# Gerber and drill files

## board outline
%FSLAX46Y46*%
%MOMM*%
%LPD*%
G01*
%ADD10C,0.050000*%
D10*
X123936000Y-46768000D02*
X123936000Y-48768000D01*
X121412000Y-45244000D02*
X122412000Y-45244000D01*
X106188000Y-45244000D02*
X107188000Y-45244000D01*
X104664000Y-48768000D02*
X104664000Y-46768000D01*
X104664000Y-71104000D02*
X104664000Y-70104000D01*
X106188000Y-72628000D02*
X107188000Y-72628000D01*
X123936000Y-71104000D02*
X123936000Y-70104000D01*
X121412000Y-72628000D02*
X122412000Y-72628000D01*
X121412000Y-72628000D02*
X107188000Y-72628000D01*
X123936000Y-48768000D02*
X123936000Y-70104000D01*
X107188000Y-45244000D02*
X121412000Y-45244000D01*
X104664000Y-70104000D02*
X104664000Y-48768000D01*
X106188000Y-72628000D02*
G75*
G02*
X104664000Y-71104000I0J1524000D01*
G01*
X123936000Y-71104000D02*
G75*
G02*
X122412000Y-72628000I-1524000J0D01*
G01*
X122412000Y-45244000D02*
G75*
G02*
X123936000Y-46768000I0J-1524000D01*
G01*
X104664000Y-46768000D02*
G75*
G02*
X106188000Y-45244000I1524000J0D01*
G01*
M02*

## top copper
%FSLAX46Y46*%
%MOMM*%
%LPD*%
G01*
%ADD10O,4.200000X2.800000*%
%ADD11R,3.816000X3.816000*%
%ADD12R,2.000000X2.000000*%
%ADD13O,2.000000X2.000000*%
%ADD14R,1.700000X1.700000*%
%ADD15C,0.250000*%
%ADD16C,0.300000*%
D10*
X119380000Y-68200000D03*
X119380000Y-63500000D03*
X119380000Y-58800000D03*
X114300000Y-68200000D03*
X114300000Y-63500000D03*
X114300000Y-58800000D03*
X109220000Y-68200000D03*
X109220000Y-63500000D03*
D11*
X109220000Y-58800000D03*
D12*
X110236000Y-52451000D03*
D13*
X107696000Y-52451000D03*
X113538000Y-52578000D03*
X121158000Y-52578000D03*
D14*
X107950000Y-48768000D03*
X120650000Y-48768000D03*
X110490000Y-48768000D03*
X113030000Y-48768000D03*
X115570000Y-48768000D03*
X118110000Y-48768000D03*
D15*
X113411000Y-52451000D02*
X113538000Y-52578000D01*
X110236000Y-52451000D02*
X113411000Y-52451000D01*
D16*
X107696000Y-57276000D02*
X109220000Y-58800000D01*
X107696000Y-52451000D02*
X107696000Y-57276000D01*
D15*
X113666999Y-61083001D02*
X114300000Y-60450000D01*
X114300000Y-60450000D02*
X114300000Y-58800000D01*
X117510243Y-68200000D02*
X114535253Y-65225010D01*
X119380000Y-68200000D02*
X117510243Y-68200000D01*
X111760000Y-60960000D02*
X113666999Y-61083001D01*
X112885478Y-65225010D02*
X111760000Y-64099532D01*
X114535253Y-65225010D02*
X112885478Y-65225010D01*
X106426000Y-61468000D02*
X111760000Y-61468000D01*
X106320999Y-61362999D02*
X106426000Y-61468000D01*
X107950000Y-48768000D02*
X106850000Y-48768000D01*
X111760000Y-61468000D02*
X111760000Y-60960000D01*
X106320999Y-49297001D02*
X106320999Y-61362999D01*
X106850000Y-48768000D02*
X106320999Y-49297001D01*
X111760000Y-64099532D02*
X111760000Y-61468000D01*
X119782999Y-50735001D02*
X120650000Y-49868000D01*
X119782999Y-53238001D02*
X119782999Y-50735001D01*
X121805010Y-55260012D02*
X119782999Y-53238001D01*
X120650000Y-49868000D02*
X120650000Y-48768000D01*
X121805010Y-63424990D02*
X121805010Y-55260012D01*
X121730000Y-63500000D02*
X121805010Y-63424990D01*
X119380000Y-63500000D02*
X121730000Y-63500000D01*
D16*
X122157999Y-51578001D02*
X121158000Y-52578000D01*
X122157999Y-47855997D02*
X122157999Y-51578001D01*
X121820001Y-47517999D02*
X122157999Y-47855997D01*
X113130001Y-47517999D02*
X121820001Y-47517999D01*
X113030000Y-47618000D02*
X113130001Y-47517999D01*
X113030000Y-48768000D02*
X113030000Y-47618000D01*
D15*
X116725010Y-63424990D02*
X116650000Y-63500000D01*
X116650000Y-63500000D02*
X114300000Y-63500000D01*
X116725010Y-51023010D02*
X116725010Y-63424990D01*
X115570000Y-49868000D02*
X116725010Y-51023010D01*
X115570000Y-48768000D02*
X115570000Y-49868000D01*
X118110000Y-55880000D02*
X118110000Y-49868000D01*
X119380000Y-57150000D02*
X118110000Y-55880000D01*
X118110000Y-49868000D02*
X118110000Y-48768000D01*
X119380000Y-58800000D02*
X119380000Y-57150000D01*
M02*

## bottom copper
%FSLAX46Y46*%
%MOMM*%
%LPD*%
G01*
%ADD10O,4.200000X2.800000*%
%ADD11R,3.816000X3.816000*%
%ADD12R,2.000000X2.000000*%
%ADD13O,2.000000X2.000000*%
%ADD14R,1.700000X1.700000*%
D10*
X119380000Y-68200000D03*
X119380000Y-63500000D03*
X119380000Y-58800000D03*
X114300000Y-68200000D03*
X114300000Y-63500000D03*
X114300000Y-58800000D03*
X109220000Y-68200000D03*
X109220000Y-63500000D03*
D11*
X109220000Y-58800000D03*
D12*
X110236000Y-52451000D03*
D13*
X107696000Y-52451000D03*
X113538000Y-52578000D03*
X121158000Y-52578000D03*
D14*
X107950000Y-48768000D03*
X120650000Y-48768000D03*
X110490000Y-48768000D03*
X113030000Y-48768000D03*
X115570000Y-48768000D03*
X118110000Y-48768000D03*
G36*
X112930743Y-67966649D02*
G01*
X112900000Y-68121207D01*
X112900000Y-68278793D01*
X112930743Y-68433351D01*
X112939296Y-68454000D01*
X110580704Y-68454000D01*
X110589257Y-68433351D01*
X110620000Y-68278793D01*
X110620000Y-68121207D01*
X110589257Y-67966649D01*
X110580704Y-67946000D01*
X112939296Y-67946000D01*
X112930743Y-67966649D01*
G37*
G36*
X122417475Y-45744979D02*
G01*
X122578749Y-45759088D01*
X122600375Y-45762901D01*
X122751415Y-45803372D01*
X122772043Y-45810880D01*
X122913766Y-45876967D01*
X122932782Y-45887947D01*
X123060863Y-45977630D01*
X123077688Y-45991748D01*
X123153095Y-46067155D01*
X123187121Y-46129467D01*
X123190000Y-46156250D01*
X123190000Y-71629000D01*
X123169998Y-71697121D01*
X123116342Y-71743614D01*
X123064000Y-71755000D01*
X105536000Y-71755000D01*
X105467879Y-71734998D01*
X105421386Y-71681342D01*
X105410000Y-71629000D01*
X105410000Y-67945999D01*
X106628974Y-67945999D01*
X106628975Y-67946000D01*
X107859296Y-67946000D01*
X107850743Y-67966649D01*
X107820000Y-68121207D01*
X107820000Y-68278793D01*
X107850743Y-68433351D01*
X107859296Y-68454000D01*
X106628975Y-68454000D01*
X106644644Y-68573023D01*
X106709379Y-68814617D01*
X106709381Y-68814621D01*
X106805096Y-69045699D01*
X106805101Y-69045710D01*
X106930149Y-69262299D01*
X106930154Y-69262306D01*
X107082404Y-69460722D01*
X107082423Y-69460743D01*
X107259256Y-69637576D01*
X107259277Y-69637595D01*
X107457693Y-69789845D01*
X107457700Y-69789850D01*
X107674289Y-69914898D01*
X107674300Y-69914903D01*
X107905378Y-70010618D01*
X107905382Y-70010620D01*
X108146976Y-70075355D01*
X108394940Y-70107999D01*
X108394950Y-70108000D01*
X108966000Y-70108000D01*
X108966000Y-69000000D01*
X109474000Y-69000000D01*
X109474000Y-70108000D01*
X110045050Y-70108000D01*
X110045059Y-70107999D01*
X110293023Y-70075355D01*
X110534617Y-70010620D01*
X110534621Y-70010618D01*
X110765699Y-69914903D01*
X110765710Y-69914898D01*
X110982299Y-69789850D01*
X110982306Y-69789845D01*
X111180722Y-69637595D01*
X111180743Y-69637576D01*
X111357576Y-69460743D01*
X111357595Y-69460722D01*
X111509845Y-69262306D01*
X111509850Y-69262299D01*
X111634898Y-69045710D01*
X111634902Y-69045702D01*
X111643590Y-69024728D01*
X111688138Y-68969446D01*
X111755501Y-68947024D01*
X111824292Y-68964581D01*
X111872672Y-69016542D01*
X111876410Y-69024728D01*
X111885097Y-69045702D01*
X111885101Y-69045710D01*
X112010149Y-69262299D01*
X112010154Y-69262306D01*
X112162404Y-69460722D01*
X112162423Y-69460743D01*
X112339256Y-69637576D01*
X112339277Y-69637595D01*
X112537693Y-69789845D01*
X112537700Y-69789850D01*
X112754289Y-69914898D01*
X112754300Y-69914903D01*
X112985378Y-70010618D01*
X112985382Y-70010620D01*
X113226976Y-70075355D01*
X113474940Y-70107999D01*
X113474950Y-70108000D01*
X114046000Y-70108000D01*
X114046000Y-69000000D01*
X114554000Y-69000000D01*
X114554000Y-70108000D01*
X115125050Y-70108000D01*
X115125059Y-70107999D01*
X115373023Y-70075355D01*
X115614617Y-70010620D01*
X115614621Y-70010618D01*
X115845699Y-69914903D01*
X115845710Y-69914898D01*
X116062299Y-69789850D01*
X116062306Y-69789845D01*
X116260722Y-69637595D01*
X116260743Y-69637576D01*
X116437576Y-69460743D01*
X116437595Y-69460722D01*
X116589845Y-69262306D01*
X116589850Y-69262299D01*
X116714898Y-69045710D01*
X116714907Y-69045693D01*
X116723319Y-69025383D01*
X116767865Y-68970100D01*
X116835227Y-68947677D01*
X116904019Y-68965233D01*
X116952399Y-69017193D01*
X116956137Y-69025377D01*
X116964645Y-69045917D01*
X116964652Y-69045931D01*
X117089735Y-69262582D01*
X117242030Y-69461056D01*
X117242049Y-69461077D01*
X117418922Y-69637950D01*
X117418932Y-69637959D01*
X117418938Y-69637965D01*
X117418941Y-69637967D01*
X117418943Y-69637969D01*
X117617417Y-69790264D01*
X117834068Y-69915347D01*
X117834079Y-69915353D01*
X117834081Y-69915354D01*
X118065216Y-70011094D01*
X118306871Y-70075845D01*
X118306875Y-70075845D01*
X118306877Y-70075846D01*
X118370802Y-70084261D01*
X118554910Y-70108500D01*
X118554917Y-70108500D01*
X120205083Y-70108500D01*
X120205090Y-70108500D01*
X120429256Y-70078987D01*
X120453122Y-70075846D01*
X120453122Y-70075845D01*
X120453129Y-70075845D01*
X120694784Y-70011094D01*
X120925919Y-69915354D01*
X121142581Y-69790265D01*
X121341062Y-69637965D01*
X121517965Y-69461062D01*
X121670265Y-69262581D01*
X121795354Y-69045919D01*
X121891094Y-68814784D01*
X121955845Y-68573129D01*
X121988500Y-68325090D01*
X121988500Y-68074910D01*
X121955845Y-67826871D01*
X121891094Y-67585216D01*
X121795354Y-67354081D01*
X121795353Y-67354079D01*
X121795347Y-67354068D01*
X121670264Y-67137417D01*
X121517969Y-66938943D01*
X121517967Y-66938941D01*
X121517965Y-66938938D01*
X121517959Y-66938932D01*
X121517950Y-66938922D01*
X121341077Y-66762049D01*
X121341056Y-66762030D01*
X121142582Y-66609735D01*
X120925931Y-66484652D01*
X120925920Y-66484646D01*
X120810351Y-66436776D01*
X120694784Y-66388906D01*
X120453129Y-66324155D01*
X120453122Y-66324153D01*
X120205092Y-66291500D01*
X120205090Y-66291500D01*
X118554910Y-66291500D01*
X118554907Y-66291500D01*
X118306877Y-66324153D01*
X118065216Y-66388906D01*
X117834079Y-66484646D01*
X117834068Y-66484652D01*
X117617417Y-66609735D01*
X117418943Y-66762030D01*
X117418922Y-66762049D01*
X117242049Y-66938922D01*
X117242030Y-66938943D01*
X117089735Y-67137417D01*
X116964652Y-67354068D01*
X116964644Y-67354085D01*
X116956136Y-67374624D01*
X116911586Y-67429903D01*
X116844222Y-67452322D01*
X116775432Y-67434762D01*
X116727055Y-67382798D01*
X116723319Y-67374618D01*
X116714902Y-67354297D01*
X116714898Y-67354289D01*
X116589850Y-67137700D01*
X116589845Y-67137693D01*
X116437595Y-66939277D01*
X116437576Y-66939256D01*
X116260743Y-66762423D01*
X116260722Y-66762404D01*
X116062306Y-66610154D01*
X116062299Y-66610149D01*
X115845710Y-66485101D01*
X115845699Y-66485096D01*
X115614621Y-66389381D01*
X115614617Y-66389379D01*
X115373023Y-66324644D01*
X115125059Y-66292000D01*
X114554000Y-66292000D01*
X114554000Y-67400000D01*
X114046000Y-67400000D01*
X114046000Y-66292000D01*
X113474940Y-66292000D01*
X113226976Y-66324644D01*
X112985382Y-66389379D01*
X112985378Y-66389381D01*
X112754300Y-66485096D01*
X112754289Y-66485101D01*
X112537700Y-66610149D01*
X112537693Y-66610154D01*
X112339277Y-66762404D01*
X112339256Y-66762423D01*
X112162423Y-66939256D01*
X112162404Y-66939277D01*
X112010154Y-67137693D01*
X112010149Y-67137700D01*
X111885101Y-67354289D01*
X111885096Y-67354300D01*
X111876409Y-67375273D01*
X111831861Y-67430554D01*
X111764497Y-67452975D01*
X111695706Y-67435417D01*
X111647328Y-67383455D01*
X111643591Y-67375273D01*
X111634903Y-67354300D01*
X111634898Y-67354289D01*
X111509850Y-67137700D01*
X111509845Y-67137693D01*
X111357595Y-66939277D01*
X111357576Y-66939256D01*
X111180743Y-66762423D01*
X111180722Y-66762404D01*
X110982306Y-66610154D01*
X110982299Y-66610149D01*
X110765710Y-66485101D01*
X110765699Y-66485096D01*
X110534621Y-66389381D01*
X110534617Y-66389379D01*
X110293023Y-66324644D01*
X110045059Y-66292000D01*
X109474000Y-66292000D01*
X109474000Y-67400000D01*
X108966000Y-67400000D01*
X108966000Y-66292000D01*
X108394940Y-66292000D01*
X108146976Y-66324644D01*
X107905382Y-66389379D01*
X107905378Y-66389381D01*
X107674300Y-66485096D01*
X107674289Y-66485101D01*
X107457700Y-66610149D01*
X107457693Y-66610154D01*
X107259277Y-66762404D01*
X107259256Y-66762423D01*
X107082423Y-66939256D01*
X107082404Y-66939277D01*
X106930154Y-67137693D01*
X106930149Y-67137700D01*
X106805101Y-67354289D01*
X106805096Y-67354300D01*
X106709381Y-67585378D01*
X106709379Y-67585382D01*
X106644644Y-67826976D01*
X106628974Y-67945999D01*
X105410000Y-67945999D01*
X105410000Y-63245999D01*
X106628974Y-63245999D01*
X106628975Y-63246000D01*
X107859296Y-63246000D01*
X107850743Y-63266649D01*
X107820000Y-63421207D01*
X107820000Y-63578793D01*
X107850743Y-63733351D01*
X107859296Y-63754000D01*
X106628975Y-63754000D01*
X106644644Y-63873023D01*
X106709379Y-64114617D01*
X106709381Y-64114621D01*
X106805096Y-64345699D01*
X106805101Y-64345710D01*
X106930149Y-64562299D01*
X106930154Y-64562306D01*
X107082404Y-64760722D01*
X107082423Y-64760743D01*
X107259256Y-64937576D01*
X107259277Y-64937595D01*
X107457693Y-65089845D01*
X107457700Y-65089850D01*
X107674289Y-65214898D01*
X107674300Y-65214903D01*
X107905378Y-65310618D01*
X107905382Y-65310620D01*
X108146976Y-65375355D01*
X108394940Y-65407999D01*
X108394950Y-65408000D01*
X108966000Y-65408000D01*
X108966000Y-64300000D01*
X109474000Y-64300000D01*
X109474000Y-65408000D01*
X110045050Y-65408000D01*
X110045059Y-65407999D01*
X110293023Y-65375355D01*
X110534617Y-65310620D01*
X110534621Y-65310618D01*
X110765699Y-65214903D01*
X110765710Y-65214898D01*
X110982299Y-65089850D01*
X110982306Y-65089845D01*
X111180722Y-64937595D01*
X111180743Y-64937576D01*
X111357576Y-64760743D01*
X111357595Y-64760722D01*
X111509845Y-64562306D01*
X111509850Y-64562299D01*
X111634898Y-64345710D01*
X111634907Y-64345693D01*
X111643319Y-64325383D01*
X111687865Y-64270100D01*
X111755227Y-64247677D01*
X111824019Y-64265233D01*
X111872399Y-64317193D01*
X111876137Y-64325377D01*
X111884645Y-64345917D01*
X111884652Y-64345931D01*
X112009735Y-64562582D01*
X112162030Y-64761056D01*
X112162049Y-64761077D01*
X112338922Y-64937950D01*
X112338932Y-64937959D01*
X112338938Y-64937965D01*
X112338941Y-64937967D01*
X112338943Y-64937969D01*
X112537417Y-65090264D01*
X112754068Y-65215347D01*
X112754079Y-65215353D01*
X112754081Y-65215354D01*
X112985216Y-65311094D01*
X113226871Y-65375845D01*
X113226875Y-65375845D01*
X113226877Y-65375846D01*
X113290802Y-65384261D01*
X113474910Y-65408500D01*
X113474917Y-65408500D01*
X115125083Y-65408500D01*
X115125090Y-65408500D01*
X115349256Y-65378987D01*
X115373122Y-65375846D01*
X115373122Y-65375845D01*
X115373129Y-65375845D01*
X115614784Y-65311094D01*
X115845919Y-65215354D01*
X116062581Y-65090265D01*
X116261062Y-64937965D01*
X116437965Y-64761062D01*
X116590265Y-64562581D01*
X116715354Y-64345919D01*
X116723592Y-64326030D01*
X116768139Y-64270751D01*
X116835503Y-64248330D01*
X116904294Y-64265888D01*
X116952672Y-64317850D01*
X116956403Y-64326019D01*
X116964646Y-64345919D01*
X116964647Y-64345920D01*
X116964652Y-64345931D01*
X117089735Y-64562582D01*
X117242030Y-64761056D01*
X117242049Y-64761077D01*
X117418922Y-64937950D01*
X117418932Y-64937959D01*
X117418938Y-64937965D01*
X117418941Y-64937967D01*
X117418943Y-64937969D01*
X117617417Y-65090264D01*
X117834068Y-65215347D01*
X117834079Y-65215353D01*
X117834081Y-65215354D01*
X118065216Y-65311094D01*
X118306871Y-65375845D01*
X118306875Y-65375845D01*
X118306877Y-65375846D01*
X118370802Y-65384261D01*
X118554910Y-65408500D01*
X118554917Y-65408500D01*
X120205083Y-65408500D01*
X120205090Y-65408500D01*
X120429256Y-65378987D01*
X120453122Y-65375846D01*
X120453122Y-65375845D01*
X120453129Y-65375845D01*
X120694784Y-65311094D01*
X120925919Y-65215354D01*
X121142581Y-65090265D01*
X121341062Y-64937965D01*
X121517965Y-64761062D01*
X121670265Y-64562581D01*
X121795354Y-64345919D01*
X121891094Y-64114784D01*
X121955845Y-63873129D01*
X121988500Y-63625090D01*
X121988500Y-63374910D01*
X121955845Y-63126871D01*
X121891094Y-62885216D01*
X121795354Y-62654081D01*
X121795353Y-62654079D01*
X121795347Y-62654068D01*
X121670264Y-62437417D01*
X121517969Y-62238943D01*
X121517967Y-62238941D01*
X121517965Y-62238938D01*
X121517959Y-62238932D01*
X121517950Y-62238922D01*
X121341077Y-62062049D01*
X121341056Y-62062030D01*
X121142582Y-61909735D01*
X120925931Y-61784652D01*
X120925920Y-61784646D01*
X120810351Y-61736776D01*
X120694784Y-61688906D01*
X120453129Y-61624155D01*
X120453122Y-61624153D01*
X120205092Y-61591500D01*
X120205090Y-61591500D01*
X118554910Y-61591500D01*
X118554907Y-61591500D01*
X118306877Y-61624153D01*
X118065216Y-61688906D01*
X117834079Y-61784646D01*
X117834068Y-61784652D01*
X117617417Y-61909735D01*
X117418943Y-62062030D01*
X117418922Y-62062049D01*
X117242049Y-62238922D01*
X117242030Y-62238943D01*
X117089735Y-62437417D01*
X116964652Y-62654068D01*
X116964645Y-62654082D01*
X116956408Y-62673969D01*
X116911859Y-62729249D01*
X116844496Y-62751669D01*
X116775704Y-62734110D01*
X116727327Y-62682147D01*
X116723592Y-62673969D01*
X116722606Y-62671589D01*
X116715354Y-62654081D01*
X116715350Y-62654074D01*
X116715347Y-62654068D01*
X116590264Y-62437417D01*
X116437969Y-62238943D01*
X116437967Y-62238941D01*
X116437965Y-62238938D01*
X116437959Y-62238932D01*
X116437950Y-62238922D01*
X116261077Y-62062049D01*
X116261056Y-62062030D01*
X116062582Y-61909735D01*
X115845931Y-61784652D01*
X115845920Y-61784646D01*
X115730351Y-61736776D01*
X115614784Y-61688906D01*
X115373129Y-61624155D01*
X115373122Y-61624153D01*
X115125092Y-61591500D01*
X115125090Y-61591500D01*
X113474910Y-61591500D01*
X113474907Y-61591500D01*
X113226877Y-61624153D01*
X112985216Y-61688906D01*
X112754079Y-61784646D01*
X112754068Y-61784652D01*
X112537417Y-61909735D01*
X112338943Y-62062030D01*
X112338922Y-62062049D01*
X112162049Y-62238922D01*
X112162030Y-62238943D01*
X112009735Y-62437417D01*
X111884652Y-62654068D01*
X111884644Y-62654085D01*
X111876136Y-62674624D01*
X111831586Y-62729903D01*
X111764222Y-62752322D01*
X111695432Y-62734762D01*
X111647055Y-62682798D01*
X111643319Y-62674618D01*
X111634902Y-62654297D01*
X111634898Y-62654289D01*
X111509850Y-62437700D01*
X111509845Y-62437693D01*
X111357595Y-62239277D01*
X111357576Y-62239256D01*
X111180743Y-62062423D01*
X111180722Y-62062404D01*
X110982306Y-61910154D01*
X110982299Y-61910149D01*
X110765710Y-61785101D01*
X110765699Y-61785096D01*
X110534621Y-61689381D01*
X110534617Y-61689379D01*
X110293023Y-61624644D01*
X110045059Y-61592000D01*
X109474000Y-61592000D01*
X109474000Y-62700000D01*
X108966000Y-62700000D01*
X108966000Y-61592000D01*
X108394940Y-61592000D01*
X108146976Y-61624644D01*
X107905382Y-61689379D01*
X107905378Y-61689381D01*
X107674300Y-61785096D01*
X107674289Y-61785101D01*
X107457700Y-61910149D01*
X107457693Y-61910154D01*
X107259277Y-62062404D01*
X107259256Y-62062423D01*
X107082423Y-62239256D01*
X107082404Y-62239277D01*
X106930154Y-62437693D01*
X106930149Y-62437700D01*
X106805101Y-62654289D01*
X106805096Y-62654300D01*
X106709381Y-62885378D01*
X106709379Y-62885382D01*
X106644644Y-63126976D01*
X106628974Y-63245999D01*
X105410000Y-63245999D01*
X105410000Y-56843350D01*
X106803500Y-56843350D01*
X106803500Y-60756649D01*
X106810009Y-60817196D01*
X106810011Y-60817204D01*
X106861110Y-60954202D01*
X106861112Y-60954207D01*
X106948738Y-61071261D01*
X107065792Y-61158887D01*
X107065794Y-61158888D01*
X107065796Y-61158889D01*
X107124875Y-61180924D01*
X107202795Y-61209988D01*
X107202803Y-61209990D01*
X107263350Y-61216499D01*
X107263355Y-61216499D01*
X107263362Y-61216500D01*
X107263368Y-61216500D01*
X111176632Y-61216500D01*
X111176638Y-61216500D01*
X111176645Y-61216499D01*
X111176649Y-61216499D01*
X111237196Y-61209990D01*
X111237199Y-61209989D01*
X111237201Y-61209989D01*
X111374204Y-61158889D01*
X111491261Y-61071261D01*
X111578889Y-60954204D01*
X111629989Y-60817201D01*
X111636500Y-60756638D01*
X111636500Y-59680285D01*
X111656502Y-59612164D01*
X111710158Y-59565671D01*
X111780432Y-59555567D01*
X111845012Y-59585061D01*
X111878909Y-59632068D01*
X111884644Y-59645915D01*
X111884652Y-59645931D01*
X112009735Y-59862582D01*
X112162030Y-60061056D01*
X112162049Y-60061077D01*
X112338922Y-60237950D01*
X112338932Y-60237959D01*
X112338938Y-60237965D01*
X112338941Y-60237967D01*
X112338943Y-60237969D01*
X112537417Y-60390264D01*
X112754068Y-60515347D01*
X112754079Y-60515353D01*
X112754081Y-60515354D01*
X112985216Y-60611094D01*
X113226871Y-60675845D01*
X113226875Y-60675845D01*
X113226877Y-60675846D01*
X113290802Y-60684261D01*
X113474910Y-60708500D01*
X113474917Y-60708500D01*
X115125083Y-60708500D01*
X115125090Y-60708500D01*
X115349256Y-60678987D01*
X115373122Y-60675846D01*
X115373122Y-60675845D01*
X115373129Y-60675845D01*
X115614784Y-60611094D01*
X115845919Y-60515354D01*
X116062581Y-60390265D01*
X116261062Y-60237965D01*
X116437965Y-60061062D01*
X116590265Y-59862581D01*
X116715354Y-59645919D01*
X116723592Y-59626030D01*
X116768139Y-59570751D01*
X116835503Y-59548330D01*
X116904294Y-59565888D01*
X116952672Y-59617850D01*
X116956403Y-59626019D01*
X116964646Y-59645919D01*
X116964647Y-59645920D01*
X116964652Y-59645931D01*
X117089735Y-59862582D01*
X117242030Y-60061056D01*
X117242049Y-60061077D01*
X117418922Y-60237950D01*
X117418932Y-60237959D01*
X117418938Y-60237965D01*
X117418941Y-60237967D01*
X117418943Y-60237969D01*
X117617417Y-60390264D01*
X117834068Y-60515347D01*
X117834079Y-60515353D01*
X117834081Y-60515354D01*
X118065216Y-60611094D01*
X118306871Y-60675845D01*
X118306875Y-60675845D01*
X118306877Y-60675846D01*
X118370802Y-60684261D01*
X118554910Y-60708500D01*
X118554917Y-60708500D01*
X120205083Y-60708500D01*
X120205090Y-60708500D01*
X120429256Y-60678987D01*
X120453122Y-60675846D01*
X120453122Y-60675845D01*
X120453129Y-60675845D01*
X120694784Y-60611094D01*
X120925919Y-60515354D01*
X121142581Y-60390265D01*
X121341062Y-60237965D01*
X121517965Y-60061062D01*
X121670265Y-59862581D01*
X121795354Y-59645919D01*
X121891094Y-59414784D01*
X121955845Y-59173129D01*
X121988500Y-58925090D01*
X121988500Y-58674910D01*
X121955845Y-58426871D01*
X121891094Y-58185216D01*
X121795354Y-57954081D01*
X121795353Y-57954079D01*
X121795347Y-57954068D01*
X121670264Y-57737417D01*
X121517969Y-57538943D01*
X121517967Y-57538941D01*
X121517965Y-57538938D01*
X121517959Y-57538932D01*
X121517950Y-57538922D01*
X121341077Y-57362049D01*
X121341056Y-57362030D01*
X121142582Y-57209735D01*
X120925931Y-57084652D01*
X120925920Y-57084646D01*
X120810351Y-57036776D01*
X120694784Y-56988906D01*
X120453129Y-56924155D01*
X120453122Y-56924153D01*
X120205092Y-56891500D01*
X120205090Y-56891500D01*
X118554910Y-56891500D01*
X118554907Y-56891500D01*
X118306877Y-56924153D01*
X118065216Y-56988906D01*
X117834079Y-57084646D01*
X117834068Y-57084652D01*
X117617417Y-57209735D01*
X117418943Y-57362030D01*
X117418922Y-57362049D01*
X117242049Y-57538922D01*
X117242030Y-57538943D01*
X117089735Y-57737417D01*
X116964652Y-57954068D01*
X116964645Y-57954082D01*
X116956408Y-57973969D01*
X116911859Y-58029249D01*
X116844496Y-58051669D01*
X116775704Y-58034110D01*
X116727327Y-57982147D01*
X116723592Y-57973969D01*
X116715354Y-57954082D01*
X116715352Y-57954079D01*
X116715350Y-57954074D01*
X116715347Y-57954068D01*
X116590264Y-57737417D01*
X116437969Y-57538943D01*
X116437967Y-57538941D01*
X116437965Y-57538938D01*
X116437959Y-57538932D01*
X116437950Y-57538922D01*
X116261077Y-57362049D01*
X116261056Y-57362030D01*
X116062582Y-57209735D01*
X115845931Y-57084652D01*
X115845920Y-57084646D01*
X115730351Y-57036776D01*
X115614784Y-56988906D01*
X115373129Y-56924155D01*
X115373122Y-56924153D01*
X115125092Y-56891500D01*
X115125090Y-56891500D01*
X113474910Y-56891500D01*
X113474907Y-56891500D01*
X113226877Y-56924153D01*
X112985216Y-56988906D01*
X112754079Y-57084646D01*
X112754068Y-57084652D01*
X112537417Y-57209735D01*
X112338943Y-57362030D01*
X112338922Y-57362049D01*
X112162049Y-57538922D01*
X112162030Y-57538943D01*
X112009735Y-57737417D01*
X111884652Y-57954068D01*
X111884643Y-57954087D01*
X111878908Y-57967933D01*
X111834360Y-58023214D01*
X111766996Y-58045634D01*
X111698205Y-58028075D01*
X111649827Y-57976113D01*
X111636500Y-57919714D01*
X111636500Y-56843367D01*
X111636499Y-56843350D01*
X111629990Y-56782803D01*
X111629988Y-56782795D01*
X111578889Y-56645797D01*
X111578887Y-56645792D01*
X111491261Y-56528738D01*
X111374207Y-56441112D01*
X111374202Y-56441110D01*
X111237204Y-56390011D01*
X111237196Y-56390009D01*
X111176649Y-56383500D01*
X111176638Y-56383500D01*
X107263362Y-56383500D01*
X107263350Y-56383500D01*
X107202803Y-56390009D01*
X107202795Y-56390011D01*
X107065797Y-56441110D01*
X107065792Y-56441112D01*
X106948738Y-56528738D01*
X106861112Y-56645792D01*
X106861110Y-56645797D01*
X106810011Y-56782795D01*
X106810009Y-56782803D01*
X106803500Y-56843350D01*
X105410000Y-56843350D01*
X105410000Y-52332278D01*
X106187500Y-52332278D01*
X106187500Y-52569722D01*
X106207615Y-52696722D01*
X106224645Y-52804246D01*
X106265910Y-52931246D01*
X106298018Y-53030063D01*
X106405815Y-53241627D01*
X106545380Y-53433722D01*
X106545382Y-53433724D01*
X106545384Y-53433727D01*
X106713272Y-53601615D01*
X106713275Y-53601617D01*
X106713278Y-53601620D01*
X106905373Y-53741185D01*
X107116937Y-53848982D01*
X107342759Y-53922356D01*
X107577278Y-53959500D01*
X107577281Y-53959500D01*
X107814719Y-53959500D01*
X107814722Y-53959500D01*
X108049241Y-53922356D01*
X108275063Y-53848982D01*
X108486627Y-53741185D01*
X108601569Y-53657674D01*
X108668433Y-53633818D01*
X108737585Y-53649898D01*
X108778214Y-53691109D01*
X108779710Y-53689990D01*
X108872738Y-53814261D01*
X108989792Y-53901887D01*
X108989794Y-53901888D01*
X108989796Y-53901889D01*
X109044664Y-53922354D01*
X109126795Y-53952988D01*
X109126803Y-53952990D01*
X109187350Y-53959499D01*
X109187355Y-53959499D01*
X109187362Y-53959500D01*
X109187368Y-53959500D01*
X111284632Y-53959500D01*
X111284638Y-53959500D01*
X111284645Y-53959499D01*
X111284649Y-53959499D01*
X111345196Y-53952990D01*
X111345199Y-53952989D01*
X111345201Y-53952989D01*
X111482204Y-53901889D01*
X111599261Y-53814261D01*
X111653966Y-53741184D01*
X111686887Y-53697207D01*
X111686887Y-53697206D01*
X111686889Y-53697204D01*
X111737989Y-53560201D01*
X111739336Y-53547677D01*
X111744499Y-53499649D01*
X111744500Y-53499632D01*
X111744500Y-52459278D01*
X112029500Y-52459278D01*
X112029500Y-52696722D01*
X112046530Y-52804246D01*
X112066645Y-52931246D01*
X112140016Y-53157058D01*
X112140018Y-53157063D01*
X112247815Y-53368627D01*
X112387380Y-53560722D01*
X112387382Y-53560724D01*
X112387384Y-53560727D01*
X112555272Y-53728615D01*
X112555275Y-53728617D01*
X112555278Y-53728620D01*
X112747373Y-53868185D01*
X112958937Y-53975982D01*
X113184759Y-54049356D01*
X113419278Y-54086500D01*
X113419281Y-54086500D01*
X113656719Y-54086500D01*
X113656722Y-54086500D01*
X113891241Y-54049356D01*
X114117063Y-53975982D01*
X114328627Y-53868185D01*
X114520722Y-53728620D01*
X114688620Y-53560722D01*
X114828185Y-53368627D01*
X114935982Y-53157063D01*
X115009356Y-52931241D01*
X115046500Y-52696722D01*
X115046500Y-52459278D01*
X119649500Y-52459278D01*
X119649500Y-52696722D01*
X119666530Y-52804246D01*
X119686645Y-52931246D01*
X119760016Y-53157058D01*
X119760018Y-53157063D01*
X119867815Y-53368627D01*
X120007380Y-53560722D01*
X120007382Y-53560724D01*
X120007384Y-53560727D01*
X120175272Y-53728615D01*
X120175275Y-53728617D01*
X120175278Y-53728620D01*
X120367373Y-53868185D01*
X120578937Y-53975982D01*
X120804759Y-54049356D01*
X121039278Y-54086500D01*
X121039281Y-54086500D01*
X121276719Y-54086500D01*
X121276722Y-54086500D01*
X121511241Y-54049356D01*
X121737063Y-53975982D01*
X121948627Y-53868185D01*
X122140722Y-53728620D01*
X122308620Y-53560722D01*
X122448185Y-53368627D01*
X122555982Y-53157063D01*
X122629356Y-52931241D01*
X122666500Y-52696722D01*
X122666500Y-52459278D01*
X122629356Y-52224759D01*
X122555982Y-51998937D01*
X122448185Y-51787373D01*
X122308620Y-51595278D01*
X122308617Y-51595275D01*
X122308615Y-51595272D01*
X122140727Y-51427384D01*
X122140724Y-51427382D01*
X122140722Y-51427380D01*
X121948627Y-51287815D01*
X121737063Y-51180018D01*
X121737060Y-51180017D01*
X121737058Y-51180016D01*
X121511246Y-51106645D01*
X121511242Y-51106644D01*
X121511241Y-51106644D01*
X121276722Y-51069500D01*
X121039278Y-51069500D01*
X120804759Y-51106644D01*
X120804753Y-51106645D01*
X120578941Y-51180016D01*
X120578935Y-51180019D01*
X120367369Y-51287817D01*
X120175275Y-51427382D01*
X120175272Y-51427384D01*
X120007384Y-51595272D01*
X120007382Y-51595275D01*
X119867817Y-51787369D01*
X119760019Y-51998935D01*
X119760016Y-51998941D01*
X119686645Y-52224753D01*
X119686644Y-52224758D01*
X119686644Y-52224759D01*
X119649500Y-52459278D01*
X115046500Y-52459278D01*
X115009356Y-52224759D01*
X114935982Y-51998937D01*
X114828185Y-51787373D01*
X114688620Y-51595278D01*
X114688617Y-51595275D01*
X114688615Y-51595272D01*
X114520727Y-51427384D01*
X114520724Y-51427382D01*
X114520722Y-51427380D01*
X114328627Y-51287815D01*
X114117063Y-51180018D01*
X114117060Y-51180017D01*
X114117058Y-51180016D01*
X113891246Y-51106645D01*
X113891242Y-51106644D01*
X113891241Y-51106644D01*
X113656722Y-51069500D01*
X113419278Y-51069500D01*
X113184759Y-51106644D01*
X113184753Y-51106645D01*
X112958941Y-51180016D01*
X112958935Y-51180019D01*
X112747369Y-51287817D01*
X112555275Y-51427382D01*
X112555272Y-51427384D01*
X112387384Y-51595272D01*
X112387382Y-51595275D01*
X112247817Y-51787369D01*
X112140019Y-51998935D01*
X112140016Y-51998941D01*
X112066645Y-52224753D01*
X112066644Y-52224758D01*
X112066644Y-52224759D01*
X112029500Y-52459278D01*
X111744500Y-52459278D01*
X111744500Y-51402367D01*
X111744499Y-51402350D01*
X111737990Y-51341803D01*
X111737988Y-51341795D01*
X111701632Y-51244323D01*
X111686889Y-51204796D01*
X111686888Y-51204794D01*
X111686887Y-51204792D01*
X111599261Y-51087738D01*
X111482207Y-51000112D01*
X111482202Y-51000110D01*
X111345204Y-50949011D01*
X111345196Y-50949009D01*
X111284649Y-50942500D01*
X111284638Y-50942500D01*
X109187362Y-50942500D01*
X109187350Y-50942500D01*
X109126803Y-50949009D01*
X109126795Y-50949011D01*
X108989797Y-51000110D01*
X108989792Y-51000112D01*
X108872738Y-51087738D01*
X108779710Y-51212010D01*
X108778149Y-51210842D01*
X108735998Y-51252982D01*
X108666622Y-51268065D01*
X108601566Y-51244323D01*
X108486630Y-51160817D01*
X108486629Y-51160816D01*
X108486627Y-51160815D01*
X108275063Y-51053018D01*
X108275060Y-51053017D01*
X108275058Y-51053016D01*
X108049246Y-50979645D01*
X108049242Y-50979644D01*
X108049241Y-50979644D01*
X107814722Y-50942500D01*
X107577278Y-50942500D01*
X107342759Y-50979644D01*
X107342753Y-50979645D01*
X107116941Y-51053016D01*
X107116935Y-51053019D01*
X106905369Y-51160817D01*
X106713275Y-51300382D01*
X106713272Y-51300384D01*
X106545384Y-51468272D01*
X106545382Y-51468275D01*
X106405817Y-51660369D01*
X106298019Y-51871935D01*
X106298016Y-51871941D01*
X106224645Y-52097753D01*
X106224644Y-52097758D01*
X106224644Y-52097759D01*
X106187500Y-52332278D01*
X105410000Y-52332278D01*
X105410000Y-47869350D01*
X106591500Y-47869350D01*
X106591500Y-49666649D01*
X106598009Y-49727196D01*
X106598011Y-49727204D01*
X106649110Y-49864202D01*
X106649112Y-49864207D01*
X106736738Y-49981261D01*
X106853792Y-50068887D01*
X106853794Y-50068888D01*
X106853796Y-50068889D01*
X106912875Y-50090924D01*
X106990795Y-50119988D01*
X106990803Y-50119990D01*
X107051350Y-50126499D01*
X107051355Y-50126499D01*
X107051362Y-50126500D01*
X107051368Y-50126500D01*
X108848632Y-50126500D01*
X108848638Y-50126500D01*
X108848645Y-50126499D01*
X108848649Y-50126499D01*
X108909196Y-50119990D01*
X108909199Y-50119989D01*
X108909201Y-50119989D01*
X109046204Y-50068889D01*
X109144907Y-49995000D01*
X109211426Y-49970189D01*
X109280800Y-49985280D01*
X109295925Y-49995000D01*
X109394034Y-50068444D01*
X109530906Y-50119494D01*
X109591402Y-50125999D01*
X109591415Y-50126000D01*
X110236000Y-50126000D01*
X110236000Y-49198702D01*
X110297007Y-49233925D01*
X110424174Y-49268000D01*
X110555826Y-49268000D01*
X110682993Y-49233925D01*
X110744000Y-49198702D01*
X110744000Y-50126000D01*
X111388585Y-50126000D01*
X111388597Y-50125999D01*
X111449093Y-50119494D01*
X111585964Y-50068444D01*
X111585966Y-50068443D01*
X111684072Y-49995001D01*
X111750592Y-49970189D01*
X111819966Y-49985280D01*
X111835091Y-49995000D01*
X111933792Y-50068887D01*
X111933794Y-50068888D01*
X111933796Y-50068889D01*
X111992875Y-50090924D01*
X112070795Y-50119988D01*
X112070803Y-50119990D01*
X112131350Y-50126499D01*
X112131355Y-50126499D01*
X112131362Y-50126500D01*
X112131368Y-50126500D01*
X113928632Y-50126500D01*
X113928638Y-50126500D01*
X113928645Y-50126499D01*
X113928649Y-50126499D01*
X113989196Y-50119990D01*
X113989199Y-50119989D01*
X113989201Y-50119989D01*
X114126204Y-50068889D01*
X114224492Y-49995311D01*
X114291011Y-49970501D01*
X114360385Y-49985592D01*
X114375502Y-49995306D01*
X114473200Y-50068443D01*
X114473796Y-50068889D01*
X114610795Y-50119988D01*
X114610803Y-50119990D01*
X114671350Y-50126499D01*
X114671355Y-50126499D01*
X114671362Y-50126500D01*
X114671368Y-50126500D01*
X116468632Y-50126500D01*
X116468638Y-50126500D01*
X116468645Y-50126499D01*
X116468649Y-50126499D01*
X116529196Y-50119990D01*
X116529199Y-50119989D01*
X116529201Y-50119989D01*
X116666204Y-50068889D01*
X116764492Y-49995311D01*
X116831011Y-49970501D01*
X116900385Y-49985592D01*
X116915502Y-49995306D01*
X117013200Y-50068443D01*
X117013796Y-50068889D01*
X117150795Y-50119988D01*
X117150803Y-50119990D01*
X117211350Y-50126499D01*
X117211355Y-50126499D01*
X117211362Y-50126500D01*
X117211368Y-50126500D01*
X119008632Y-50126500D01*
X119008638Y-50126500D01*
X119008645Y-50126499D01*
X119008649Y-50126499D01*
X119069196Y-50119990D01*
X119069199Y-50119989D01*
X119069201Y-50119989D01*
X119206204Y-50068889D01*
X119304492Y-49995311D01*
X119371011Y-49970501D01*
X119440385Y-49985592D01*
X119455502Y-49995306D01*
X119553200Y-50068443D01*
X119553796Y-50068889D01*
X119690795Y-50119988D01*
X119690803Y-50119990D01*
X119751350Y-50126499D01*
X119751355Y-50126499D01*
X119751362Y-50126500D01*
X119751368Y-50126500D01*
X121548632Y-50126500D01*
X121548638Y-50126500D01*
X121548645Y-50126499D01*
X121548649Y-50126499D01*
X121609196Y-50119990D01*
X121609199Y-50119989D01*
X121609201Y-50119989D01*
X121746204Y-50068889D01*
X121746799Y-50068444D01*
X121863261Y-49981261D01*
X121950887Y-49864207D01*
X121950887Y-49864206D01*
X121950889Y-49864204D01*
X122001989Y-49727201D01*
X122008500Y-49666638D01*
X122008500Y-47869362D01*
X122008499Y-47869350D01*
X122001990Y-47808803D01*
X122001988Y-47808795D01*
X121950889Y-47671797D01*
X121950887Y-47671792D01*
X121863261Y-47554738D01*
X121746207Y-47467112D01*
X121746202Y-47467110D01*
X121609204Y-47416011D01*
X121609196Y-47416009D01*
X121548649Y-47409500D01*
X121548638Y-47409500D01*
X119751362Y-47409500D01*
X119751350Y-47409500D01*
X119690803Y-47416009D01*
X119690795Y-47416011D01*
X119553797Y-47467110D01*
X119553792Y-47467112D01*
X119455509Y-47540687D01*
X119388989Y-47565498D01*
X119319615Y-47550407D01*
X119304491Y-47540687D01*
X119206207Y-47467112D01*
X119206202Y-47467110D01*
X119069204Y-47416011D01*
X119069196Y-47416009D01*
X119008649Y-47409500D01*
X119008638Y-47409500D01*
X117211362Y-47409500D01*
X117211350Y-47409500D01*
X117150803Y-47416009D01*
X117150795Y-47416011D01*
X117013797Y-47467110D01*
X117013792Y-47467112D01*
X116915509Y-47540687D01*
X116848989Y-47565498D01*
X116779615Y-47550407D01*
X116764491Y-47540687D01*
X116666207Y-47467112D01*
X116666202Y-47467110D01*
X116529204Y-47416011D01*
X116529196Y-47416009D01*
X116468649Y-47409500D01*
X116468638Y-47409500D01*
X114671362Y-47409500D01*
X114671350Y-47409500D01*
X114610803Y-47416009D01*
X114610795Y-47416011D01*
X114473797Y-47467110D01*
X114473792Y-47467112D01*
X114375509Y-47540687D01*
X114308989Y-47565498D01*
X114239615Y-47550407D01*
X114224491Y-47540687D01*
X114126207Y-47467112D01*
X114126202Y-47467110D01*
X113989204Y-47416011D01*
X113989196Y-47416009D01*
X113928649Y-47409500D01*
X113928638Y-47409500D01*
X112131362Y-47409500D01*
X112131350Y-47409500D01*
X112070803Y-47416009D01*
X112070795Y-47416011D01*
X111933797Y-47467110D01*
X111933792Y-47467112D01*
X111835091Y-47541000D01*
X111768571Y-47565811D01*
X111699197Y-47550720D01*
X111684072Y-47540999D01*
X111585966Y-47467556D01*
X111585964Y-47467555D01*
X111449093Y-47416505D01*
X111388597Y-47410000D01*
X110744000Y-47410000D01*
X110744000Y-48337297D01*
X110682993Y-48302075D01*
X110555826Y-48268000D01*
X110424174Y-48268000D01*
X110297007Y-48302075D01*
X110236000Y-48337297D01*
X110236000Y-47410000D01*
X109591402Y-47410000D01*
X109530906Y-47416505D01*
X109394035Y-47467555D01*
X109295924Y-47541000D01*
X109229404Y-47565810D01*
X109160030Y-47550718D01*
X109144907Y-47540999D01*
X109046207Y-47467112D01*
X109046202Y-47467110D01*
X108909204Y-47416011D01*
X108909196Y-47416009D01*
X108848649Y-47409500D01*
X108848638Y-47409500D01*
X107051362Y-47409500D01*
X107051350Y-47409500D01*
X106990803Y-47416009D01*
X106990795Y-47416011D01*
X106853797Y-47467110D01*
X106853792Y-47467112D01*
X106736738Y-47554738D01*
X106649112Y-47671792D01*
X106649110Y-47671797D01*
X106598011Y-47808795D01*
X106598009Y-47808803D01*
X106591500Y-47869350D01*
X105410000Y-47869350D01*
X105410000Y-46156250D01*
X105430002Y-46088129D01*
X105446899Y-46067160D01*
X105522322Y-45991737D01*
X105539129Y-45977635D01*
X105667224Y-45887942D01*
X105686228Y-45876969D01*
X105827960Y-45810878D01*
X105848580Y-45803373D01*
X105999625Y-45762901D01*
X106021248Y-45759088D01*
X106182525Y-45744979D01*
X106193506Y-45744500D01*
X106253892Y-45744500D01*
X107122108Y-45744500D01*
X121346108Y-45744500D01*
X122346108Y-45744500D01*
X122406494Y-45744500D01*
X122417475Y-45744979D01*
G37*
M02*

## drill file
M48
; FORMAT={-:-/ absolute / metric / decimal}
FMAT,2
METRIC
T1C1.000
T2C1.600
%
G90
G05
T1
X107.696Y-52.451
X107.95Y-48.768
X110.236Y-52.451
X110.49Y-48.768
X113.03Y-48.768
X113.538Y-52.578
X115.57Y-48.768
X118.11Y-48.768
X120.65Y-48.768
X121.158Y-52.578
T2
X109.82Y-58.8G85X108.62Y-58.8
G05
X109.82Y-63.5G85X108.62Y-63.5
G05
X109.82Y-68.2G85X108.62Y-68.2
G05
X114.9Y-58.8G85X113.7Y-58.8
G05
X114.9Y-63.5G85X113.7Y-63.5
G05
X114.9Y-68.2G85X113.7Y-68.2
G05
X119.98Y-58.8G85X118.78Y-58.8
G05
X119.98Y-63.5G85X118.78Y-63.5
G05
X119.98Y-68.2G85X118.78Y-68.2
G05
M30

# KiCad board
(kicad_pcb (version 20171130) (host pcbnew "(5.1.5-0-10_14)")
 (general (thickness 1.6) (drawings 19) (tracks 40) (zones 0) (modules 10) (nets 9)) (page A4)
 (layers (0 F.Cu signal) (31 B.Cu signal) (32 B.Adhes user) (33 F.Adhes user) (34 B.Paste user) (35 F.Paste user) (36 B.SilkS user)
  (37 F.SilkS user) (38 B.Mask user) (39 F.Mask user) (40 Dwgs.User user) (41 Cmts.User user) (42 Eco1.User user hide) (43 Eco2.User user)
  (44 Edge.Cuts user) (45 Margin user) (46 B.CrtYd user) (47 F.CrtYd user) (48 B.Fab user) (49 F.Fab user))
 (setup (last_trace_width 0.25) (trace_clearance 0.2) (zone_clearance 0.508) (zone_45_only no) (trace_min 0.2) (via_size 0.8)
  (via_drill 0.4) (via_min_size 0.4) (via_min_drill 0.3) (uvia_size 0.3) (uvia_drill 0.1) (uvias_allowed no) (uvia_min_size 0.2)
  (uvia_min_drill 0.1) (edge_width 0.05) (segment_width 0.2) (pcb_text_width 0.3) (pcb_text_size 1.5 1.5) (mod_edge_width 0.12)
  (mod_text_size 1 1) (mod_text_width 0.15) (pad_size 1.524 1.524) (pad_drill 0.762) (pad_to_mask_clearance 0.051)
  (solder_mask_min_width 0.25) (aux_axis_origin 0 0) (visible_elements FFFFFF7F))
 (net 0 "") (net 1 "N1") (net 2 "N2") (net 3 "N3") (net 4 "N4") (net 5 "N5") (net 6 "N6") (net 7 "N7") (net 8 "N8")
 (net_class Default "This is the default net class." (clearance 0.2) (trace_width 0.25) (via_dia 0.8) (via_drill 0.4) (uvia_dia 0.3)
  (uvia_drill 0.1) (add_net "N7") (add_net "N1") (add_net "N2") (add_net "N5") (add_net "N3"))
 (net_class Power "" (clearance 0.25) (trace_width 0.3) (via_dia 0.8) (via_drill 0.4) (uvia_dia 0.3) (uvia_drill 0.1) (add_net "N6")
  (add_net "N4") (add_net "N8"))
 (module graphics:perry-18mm (layer F.Cu) (at 114.3 62.23)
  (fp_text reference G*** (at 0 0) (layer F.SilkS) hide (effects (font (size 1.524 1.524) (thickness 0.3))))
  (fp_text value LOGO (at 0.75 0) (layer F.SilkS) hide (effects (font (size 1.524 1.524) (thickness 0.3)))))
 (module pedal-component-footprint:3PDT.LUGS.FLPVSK (layer F.Cu) (at 114.3 63.5)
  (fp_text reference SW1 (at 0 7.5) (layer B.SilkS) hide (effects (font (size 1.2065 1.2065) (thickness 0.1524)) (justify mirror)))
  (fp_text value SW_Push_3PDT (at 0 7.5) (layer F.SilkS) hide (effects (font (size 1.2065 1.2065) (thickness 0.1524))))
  (pad 9 thru_hole oval (at 5.08 4.7 180) (size 4.2 2.8) (drill oval 2.8 1.6) (layers *.Cu *.Mask) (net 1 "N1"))
  (pad 8 thru_hole oval (at 5.08 0 180) (size 4.2 2.8) (drill oval 2.8 1.6) (layers *.Cu *.Mask) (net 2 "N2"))
  (pad 7 thru_hole oval (at 5.08 -4.7 180) (size 4.2 2.8) (drill oval 2.8 1.6) (layers *.Cu *.Mask) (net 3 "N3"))
  (pad 6 thru_hole oval (at 0 4.7 180) (size 4.2 2.8) (drill oval 2.8 1.6) (layers *.Cu *.Mask) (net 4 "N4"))
  (pad 5 thru_hole oval (at 0 0 180) (size 4.2 2.8) (drill oval 2.8 1.6) (layers *.Cu *.Mask) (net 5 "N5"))
  (pad 4 thru_hole oval (at 0 -4.7 180) (size 4.2 2.8) (drill oval 2.8 1.6) (layers *.Cu *.Mask) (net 1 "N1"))
  (pad 3 thru_hole oval (at -5.08 4.7 180) (size 4.2 2.8) (drill oval 2.8 1.6) (layers *.Cu *.Mask) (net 4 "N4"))
  (pad 2 thru_hole oval (at -5.08 0 180) (size 4.2 2.8) (drill oval 2.8 1.6) (layers *.Cu *.Mask) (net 4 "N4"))
  (pad 1 thru_hole rect (at -5.08 -4.7 180) (size 3.816 3.816) (drill oval 2.8 1.6) (layers *.Cu *.Mask) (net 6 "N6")))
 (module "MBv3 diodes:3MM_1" (layer F.Cu) (at 108.966 52.451 180)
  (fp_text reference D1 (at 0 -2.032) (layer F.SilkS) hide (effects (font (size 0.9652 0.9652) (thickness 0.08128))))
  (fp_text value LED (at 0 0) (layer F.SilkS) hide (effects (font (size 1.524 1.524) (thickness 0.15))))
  (pad 2 thru_hole rect (at -1.27 0 180) (size 2 2) (drill 1) (layers *.Cu *.Mask) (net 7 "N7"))
  (pad 1 thru_hole oval (at 1.27 0 180) (size 2 2) (drill 1) (layers *.Cu *.Mask) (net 6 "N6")))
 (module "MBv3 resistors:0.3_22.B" (layer F.Cu) (at 117.348 52.578)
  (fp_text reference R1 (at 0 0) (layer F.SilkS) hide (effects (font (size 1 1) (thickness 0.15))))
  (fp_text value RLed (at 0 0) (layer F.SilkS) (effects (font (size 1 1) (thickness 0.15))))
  (pad 1 thru_hole oval (at -3.81 0) (size 2 2) (drill 1) (layers *.Cu *.Mask) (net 7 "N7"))
  (pad 2 thru_hole oval (at 3.81 0) (size 2 2) (drill 1) (layers *.Cu *.Mask) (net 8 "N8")))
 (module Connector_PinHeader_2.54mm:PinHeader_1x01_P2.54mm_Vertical (layer F.Cu) (at 107.95 48.768 180)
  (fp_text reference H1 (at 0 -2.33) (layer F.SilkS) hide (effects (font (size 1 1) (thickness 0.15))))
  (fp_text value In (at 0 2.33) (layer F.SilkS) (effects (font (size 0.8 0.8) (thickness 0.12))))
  (pad 1 thru_hole rect (at 0 0 180) (size 1.7 1.7) (drill 1) (layers *.Cu *.Mask) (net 1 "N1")))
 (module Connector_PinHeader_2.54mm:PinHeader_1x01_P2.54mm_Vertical (layer F.Cu) (at 120.65 48.768 180)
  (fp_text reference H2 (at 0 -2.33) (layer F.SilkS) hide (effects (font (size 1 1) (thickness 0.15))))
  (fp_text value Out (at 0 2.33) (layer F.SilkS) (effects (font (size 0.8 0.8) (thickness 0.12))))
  (pad 1 thru_hole rect (at 0 0 180) (size 1.7 1.7) (drill 1) (layers *.Cu *.Mask) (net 2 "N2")))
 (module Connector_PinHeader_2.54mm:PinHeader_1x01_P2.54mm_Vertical (layer F.Cu) (at 110.49 48.768 180)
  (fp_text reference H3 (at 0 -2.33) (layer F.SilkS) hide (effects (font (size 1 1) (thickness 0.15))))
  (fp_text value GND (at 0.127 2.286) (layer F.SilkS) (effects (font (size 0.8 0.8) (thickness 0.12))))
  (pad 1 thru_hole rect (at 0 0 180) (size 1.7 1.7) (drill 1) (layers *.Cu *.Mask) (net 4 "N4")))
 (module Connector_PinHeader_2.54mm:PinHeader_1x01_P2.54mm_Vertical (layer F.Cu) (at 113.03 48.768 180)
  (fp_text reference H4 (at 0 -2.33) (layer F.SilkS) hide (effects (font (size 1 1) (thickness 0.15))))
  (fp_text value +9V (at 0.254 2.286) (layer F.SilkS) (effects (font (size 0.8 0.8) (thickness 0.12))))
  (pad 1 thru_hole rect (at 0 0 180) (size 1.7 1.7) (drill 1) (layers *.Cu *.Mask) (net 8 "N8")))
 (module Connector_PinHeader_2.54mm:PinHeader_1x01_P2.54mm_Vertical (layer F.Cu) (at 115.57 48.768 180)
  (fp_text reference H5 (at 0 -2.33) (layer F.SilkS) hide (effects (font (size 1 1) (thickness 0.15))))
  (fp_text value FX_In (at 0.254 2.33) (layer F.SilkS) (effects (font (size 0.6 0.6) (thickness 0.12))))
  (pad 1 thru_hole rect (at 0 0 180) (size 1.7 1.7) (drill 1) (layers *.Cu *.Mask) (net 5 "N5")))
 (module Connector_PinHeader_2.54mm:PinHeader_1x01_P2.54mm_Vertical (layer F.Cu) (at 118.11 48.768 180)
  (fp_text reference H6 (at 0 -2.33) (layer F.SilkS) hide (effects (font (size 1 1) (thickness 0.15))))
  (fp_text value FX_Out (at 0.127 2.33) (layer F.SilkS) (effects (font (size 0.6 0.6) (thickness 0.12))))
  (pad 1 thru_hole rect (at 0 0 180) (size 1.7 1.7) (drill 1) (layers *.Cu *.Mask) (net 3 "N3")))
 (gr_line (start 123.936 46.768) (end 123.936 48.768) (layer Edge.Cuts) (width 0.05))
 (gr_line (start 121.412 45.244) (end 122.412 45.244) (layer Edge.Cuts) (width 0.05))
 (gr_line (start 106.188 45.244) (end 107.188 45.244) (layer Edge.Cuts) (width 0.05))
 (gr_line (start 104.664 48.768) (end 104.664 46.768) (layer Edge.Cuts) (width 0.05))
 (gr_line (start 104.664 71.104) (end 104.664 70.104) (layer Edge.Cuts) (width 0.05))
 (gr_line (start 106.188 72.628) (end 107.188 72.628) (layer Edge.Cuts) (width 0.05))
 (gr_line (start 123.936 71.104) (end 123.936 70.104) (layer Edge.Cuts) (width 0.05))
 (gr_line (start 121.412 72.628) (end 122.412 72.628) (layer Edge.Cuts) (width 0.05))
 (gr_line (start 121.412 72.628) (end 107.188 72.628) (layer Edge.Cuts) (width 0.05))
 (gr_line (start 123.936 48.768) (end 123.936 70.104) (layer Edge.Cuts) (width 0.05))
 (gr_line (start 107.188 45.244) (end 121.412 45.244) (layer Edge.Cuts) (width 0.05))
 (gr_line (start 104.664 70.104) (end 104.664 48.768) (layer Edge.Cuts) (width 0.05))
 (gr_arc (start 106.188 71.104) (end 104.664 71.104) (angle -90) (layer Edge.Cuts) (width 0.05))
 (gr_arc (start 122.412 71.104) (end 122.412 72.628) (angle -90) (layer Edge.Cuts) (width 0.05))
 (gr_arc (start 122.412 46.768) (end 123.936 46.768) (angle -90) (layer Edge.Cuts) (width 0.05))
 (gr_arc (start 106.188 46.768) (end 106.188 45.244) (angle -90) (layer Edge.Cuts) (width 0.05))
 (segment (start 113.411 52.451) (end 113.538 52.578) (width 0.25) (layer F.Cu) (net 7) (status 30))
 (segment (start 110.236 52.451) (end 113.411 52.451) (width 0.25) (layer F.Cu) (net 7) (status 30))
 (segment (start 107.696 57.276) (end 109.22 58.8) (width 0.3) (layer F.Cu) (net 6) (status 30))
 (segment (start 107.696 52.451) (end 107.696 57.276) (width 0.3) (layer F.Cu) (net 6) (status 30))
 (segment (start 113.666999 61.083001) (end 114.3 60.45) (width 0.25) (layer F.Cu) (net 1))
 (segment (start 114.3 60.45) (end 114.3 58.8) (width 0.25) (layer F.Cu) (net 1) (status 20))
 (segment (start 117.510243 68.2) (end 114.535253 65.22501) (width 0.25) (layer F.Cu) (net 1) (status 10))
 (segment (start 119.38 68.2) (end 117.510243 68.2) (width 0.25) (layer F.Cu) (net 1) (status 30))
 (segment (start 111.76 60.96) (end 113.666999 61.083001) (width 0.25) (layer F.Cu) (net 1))
 (segment (start 112.885478 65.22501) (end 111.76 64.099532) (width 0.25) (layer F.Cu) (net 1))
 (segment (start 114.535253 65.22501) (end 112.885478 65.22501) (width 0.25) (layer F.Cu) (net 1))
 (segment (start 106.426 61.468) (end 111.76 61.468) (width 0.25) (layer F.Cu) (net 1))
 (segment (start 106.320999 61.362999) (end 106.426 61.468) (width 0.25) (layer F.Cu) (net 1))
 (segment (start 107.95 48.768) (end 106.85 48.768) (width 0.25) (layer F.Cu) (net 1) (status 10))
 (segment (start 111.76 61.468) (end 111.76 60.96) (width 0.25) (layer F.Cu) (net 1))
 (segment (start 106.320999 49.297001) (end 106.320999 61.362999) (width 0.25) (layer F.Cu) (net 1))
 (segment (start 106.85 48.768) (end 106.320999 49.297001) (width 0.25) (layer F.Cu) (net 1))
 (segment (start 111.76 64.099532) (end 111.76 61.468) (width 0.25) (layer F.Cu) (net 1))
 (segment (start 119.782999 50.735001) (end 120.65 49.868) (width 0.25) (layer F.Cu) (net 2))
 (segment (start 119.782999 53.238001) (end 119.782999 50.735001) (width 0.25) (layer F.Cu) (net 2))
 (segment (start 121.80501 55.260012) (end 119.782999 53.238001) (width 0.25) (layer F.Cu) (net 2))
 (segment (start 120.65 49.868) (end 120.65 48.768) (width 0.25) (layer F.Cu) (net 2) (status 20))
 (segment (start 121.80501 63.42499) (end 121.80501 55.260012) (width 0.25) (layer F.Cu) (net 2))
 (segment (start 121.73 63.5) (end 121.80501 63.42499) (width 0.25) (layer F.Cu) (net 2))
 (segment (start 119.38 63.5) (end 121.73 63.5) (width 0.25) (layer F.Cu) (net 2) (status 10))
 (segment (start 122.157999 51.578001) (end 121.158 52.578) (width 0.3) (layer F.Cu) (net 8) (status 20))
 (segment (start 122.157999 47.855997) (end 122.157999 51.578001) (width 0.3) (layer F.Cu) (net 8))
 (segment (start 121.820001 47.517999) (end 122.157999 47.855997) (width 0.3) (layer F.Cu) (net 8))
 (segment (start 113.130001 47.517999) (end 121.820001 47.517999) (width 0.3) (layer F.Cu) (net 8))
 (segment (start 113.03 47.618) (end 113.130001 47.517999) (width 0.3) (layer F.Cu) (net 8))
 (segment (start 113.03 48.768) (end 113.03 47.618) (width 0.3) (layer F.Cu) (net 8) (status 10))
 (segment (start 116.72501 63.42499) (end 116.65 63.5) (width 0.25) (layer F.Cu) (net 5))
 (segment (start 116.65 63.5) (end 114.3 63.5) (width 0.25) (layer F.Cu) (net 5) (status 20))
 (segment (start 116.72501 51.02301) (end 116.72501 63.42499) (width 0.25) (layer F.Cu) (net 5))
 (segment (start 115.57 49.868) (end 116.72501 51.02301) (width 0.25) (layer F.Cu) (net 5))
 (segment (start 115.57 48.768) (end 115.57 49.868) (width 0.25) (layer F.Cu) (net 5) (status 10))
 (segment (start 118.11 55.88) (end 118.11 49.868) (width 0.25) (layer F.Cu) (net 3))
 (segment (start 119.38 57.15) (end 118.11 55.88) (width 0.25) (layer F.Cu) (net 3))
 (segment (start 118.11 49.868) (end 118.11 48.768) (width 0.25) (layer F.Cu) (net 3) (status 20))
 (segment (start 119.38 58.8) (end 119.38 57.15) (width 0.25) (layer F.Cu) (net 3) (status 10))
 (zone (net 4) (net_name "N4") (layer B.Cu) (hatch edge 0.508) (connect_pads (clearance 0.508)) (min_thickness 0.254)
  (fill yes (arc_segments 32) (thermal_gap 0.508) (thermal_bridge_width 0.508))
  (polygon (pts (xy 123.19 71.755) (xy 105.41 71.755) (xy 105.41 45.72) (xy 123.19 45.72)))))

